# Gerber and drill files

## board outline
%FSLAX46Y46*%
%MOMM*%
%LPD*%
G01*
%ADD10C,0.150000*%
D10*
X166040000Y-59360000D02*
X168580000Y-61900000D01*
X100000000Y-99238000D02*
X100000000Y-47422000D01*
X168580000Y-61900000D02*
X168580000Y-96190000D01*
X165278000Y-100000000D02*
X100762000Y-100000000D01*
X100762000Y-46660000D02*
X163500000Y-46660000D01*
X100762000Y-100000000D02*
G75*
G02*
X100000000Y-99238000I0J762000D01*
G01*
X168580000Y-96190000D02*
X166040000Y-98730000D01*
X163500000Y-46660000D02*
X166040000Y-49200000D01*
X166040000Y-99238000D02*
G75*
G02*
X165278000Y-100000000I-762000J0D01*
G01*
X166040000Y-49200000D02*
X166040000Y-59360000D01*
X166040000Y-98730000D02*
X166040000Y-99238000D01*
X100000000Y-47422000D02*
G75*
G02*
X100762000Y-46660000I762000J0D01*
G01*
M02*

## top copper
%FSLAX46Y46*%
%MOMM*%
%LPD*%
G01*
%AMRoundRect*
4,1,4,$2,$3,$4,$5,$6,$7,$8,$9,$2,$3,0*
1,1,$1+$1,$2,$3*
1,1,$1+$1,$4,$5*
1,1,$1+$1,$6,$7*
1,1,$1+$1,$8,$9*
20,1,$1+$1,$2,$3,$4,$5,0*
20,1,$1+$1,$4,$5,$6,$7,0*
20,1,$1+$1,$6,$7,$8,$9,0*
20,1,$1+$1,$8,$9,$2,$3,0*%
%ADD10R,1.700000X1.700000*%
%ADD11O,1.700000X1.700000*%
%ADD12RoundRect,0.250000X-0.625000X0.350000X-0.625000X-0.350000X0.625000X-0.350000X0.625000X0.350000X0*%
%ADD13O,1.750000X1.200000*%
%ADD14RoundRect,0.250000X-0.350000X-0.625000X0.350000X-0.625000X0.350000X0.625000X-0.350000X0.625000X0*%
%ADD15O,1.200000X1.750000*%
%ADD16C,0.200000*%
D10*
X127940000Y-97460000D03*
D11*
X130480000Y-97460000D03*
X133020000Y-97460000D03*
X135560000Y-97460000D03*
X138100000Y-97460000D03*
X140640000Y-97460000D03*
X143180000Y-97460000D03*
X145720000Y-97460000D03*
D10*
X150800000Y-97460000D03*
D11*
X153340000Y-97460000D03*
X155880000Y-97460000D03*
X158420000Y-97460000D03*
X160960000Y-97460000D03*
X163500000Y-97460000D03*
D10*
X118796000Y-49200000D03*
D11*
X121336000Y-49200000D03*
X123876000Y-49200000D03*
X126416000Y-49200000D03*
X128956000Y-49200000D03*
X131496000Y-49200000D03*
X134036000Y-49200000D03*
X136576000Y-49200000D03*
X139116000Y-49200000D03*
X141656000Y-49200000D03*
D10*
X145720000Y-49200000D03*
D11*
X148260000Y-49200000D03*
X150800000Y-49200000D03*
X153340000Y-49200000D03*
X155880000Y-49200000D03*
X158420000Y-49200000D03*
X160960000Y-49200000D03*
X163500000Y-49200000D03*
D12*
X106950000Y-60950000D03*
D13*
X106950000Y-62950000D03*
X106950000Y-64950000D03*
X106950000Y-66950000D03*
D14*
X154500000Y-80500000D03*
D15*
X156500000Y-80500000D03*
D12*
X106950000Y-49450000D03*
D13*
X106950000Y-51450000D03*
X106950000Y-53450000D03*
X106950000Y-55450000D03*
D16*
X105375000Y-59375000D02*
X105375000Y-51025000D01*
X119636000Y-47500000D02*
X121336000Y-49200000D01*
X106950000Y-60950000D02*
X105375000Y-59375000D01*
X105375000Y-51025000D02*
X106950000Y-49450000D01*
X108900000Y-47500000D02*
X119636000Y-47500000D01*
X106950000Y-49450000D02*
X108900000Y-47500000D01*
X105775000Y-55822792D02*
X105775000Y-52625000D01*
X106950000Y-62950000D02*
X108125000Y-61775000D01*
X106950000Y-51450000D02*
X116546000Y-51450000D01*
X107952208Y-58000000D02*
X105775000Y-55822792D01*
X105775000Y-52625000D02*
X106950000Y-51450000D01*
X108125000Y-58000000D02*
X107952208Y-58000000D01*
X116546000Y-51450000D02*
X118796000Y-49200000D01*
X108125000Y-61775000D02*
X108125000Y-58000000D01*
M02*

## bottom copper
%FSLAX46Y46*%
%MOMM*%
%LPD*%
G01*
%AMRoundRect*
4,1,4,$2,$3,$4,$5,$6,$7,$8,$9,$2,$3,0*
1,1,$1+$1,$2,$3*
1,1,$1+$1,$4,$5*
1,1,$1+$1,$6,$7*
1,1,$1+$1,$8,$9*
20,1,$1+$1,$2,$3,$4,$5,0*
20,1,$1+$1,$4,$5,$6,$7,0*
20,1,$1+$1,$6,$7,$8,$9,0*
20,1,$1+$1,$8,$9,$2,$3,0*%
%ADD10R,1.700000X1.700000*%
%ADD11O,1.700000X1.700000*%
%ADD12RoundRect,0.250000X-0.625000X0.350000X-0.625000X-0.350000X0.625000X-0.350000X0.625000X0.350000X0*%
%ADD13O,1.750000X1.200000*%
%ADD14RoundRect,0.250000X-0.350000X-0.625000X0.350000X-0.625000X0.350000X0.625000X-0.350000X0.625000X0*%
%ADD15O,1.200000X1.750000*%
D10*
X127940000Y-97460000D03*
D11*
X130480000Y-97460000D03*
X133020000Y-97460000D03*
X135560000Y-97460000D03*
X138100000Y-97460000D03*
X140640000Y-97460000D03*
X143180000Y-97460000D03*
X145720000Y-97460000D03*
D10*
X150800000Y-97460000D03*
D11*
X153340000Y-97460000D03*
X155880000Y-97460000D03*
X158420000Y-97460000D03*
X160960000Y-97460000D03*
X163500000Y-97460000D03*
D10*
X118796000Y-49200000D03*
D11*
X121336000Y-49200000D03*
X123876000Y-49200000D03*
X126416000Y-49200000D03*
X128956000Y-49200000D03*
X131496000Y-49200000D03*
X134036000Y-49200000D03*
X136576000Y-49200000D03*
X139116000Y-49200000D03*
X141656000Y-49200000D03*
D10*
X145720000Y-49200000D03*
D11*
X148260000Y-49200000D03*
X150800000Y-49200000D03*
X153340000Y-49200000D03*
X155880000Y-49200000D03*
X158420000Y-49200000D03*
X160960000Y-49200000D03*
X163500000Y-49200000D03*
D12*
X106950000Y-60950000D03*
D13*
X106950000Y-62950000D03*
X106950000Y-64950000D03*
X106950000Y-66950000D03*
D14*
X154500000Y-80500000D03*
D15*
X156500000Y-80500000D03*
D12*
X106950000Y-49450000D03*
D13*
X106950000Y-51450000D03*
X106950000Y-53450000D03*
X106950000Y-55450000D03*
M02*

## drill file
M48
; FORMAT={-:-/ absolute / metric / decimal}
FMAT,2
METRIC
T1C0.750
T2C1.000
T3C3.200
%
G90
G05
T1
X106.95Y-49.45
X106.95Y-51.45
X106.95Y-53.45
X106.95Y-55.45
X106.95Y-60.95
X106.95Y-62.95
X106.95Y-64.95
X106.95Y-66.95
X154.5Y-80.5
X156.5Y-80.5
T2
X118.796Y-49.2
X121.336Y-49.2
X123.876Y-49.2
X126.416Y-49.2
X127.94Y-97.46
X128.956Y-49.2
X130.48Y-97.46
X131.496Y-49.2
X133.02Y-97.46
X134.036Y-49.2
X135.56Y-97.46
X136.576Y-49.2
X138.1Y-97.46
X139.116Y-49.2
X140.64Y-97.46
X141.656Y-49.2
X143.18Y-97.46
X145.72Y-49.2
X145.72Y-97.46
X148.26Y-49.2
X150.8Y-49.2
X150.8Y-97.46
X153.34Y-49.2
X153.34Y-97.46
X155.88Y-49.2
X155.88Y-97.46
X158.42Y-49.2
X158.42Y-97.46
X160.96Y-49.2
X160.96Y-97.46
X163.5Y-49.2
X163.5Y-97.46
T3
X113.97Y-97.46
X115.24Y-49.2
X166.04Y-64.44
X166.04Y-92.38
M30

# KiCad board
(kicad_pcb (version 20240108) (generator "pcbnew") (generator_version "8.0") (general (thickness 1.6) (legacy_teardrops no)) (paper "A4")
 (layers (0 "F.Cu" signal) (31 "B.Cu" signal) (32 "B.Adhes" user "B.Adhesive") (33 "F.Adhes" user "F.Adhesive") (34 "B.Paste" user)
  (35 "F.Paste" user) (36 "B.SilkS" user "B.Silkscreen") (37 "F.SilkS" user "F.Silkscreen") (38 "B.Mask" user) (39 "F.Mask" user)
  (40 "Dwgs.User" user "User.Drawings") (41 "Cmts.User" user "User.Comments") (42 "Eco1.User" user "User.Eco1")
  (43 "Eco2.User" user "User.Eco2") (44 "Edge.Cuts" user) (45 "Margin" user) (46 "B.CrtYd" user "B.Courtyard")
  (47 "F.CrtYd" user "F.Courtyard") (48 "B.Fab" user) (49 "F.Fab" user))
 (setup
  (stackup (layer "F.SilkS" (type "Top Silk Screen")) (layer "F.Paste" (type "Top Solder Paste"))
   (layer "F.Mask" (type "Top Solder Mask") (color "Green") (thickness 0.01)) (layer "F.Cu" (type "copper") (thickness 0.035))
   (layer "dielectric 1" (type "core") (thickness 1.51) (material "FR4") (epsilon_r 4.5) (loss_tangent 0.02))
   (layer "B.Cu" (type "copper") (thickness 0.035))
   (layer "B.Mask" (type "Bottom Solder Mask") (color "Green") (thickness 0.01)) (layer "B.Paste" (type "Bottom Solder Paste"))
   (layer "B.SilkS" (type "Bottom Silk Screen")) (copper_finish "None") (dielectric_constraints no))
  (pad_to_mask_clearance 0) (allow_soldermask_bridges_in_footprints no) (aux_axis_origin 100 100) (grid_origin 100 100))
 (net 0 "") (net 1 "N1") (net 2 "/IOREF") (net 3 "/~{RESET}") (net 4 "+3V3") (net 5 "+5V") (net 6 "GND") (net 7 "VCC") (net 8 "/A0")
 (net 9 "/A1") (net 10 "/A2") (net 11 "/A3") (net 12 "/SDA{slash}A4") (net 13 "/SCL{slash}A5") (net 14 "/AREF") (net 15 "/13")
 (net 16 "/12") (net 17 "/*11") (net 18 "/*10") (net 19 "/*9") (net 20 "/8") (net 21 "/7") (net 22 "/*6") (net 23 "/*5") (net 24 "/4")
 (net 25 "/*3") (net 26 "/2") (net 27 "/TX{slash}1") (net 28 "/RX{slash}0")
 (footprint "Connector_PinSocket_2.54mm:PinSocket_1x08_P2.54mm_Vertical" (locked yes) (layer "F.Cu") (at 127.94 97.46 90)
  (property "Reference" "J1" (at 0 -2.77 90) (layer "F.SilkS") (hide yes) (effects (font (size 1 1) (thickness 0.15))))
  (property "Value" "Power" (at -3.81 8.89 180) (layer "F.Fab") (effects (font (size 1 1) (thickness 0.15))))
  (pad "1" thru_hole rect (at 0 0 90) (size 1.7 1.7) (drill 1) (layers "*.Cu" "*.Mask") (remove_unused_layers no) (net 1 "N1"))
  (pad "2" thru_hole oval (at 0 2.54 90) (size 1.7 1.7) (drill 1) (layers "*.Cu" "*.Mask") (remove_unused_layers no) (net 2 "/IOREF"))
  (pad "3" thru_hole oval (at 0 5.08 90) (size 1.7 1.7) (drill 1) (layers "*.Cu" "*.Mask") (remove_unused_layers no) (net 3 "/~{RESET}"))
  (pad "4" thru_hole oval (at 0 7.62 90) (size 1.7 1.7) (drill 1) (layers "*.Cu" "*.Mask") (remove_unused_layers no) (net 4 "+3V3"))
  (pad "5" thru_hole oval (at 0 10.16 90) (size 1.7 1.7) (drill 1) (layers "*.Cu" "*.Mask") (remove_unused_layers no) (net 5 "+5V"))
  (pad "6" thru_hole oval (at 0 12.7 90) (size 1.7 1.7) (drill 1) (layers "*.Cu" "*.Mask") (remove_unused_layers no) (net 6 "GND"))
  (pad "7" thru_hole oval (at 0 15.24 90) (size 1.7 1.7) (drill 1) (layers "*.Cu" "*.Mask") (remove_unused_layers no) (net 6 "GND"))
  (pad "8" thru_hole oval (at 0 17.78 90) (size 1.7 1.7) (drill 1) (layers "*.Cu" "*.Mask") (remove_unused_layers no) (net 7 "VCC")))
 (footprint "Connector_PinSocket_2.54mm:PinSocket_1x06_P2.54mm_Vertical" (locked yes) (layer "F.Cu") (at 150.8 97.46 90)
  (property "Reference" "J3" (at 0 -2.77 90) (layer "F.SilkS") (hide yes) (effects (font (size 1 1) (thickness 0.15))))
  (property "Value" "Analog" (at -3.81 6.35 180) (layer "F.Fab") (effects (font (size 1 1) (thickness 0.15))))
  (pad "1" thru_hole rect (at 0 0 90) (size 1.7 1.7) (drill 1) (layers "*.Cu" "*.Mask") (remove_unused_layers no) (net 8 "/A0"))
  (pad "2" thru_hole oval (at 0 2.54 90) (size 1.7 1.7) (drill 1) (layers "*.Cu" "*.Mask") (remove_unused_layers no) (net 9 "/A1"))
  (pad "3" thru_hole oval (at 0 5.08 90) (size 1.7 1.7) (drill 1) (layers "*.Cu" "*.Mask") (remove_unused_layers no) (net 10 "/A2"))
  (pad "4" thru_hole oval (at 0 7.62 90) (size 1.7 1.7) (drill 1) (layers "*.Cu" "*.Mask") (remove_unused_layers no) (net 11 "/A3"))
  (pad "5" thru_hole oval (at 0 10.16 90) (size 1.7 1.7) (drill 1) (layers "*.Cu" "*.Mask") (remove_unused_layers no)
   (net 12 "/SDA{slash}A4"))
  (pad "6" thru_hole oval (at 0 12.7 90) (size 1.7 1.7) (drill 1) (layers "*.Cu" "*.Mask") (remove_unused_layers no)
   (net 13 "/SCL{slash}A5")))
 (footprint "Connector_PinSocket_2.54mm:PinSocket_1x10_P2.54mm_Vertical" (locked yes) (layer "F.Cu") (at 118.796 49.2 90)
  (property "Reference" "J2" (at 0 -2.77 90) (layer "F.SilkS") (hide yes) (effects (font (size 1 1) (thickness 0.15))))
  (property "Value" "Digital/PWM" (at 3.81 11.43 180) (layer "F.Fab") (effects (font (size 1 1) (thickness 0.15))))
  (pad "1" thru_hole rect (at 0 0 90) (size 1.7 1.7) (drill 1) (layers "*.Cu" "*.Mask") (remove_unused_layers no) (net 13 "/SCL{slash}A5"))
  (pad "2" thru_hole oval (at 0 2.54 90) (size 1.7 1.7) (drill 1) (layers "*.Cu" "*.Mask") (remove_unused_layers no)
   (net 12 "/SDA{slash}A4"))
  (pad "3" thru_hole oval (at 0 5.08 90) (size 1.7 1.7) (drill 1) (layers "*.Cu" "*.Mask") (remove_unused_layers no) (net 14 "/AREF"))
  (pad "4" thru_hole oval (at 0 7.62 90) (size 1.7 1.7) (drill 1) (layers "*.Cu" "*.Mask") (remove_unused_layers no) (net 6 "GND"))
  (pad "5" thru_hole oval (at 0 10.16 90) (size 1.7 1.7) (drill 1) (layers "*.Cu" "*.Mask") (remove_unused_layers no) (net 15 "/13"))
  (pad "6" thru_hole oval (at 0 12.7 90) (size 1.7 1.7) (drill 1) (layers "*.Cu" "*.Mask") (remove_unused_layers no) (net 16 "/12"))
  (pad "7" thru_hole oval (at 0 15.24 90) (size 1.7 1.7) (drill 1) (layers "*.Cu" "*.Mask") (remove_unused_layers no) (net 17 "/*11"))
  (pad "8" thru_hole oval (at 0 17.78 90) (size 1.7 1.7) (drill 1) (layers "*.Cu" "*.Mask") (remove_unused_layers no) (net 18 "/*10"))
  (pad "9" thru_hole oval (at 0 20.32 90) (size 1.7 1.7) (drill 1) (layers "*.Cu" "*.Mask") (remove_unused_layers no) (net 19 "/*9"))
  (pad "10" thru_hole oval (at 0 22.86 90) (size 1.7 1.7) (drill 1) (layers "*.Cu" "*.Mask") (remove_unused_layers no) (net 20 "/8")))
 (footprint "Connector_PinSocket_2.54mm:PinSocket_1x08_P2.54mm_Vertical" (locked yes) (layer "F.Cu") (at 145.72 49.2 90)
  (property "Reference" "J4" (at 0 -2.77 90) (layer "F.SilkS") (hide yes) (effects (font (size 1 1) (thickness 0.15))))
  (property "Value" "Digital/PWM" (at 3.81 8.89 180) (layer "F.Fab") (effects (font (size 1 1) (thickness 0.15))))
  (pad "1" thru_hole rect (at 0 0 90) (size 1.7 1.7) (drill 1) (layers "*.Cu" "*.Mask") (remove_unused_layers no) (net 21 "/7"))
  (pad "2" thru_hole oval (at 0 2.54 90) (size 1.7 1.7) (drill 1) (layers "*.Cu" "*.Mask") (remove_unused_layers no) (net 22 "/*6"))
  (pad "3" thru_hole oval (at 0 5.08 90) (size 1.7 1.7) (drill 1) (layers "*.Cu" "*.Mask") (remove_unused_layers no) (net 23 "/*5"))
  (pad "4" thru_hole oval (at 0 7.62 90) (size 1.7 1.7) (drill 1) (layers "*.Cu" "*.Mask") (remove_unused_layers no) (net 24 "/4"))
  (pad "5" thru_hole oval (at 0 10.16 90) (size 1.7 1.7) (drill 1) (layers "*.Cu" "*.Mask") (remove_unused_layers no) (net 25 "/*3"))
  (pad "6" thru_hole oval (at 0 12.7 90) (size 1.7 1.7) (drill 1) (layers "*.Cu" "*.Mask") (remove_unused_layers no) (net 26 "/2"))
  (pad "7" thru_hole oval (at 0 15.24 90) (size 1.7 1.7) (drill 1) (layers "*.Cu" "*.Mask") (remove_unused_layers no) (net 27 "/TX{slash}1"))
  (pad "8" thru_hole oval (at 0 17.78 90) (size 1.7 1.7) (drill 1) (layers "*.Cu" "*.Mask") (remove_unused_layers no) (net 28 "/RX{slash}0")))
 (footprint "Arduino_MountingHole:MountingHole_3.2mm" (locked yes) (layer "F.Cu") (at 115.24 49.2)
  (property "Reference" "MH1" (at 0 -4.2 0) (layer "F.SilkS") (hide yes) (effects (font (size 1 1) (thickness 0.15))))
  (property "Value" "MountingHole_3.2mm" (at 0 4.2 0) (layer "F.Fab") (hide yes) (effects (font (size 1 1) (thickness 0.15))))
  (pad "" np_thru_hole circle (at 0 0) (size 3.2 3.2) (drill 3.2) (layers "*.Cu" "*.Mask")))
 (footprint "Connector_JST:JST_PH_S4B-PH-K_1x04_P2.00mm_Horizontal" (layer "F.Cu") (at 106.95 60.95 -90)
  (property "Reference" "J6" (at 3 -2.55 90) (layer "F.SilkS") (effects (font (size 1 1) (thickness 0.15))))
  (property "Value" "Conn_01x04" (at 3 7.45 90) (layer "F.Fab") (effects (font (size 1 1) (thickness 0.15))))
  (pad "1" thru_hole roundrect (at 0 0 270) (size 1.2 1.75) (drill 0.75) (layers "*.Cu" "*.Mask") (remove_unused_layers no)
   (roundrect_rratio 0.208333) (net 12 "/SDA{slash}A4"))
  (pad "2" thru_hole oval (at 2 0 270) (size 1.2 1.75) (drill 0.75) (layers "*.Cu" "*.Mask") (remove_unused_layers no)
   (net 13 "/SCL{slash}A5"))
  (pad "3" thru_hole oval (at 4 0 270) (size 1.2 1.75) (drill 0.75) (layers "*.Cu" "*.Mask") (remove_unused_layers no) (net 7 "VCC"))
  (pad "4" thru_hole oval (at 6 0 270) (size 1.2 1.75) (drill 0.75) (layers "*.Cu" "*.Mask") (remove_unused_layers no) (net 6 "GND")))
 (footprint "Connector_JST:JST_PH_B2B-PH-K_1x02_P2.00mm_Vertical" (layer "F.Cu") (at 154.5 80.5)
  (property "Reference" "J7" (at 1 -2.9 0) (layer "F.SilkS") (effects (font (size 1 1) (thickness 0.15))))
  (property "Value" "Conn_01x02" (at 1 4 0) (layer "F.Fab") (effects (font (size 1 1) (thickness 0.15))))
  (pad "1" thru_hole roundrect (at 0 0) (size 1.2 1.75) (drill 0.75) (layers "*.Cu" "*.Mask") (remove_unused_layers no)
   (roundrect_rratio 0.208333) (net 6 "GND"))
  (pad "2" thru_hole oval (at 2 0) (size 1.2 1.75) (drill 0.75) (layers "*.Cu" "*.Mask") (remove_unused_layers no) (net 7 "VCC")))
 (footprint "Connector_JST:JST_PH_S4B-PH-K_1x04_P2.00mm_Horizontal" (layer "F.Cu") (at 106.95 49.45 -90)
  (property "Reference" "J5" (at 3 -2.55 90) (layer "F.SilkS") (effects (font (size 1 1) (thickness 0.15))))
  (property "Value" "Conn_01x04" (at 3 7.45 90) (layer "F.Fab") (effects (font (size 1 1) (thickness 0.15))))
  (pad "1" thru_hole roundrect (at 0 0 270) (size 1.2 1.75) (drill 0.75) (layers "*.Cu" "*.Mask") (remove_unused_layers no)
   (roundrect_rratio 0.208333) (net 12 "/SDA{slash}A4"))
  (pad "2" thru_hole oval (at 2 0 270) (size 1.2 1.75) (drill 0.75) (layers "*.Cu" "*.Mask") (remove_unused_layers no)
   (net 13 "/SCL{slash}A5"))
  (pad "3" thru_hole oval (at 4 0 270) (size 1.2 1.75) (drill 0.75) (layers "*.Cu" "*.Mask") (remove_unused_layers no) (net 7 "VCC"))
  (pad "4" thru_hole oval (at 6 0 270) (size 1.2 1.75) (drill 0.75) (layers "*.Cu" "*.Mask") (remove_unused_layers no) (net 6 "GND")))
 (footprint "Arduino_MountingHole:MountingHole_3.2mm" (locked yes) (layer "F.Cu") (at 113.97 97.46)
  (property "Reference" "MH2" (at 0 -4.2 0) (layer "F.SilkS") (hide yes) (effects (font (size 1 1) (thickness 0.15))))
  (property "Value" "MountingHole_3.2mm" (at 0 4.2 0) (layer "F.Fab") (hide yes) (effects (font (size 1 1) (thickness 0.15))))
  (pad "" np_thru_hole circle (at 0 0) (size 3.2 3.2) (drill 3.2) (layers "*.Cu" "*.Mask")))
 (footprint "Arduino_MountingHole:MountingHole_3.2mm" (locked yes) (layer "F.Cu") (at 166.04 64.44)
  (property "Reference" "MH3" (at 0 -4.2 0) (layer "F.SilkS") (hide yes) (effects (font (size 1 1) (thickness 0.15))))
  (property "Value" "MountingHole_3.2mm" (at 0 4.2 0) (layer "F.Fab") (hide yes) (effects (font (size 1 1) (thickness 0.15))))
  (pad "" np_thru_hole circle (at 0 0) (size 3.2 3.2) (drill 3.2) (layers "*.Cu" "*.Mask")))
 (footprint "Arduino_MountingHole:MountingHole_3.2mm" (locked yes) (layer "F.Cu") (at 166.04 92.38)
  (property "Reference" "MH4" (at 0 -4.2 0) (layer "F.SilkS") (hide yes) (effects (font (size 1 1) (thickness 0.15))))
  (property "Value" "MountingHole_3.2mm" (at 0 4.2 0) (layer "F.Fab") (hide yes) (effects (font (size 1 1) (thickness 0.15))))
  (pad "" np_thru_hole circle (at 0 0) (size 3.2 3.2) (drill 3.2) (layers "*.Cu" "*.Mask")))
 (gr_line (start 166.04 59.36) (end 168.58 61.9) (stroke (width 0.15) (type solid)) (layer "Edge.Cuts"))
 (gr_line (start 100 99.238) (end 100 47.422) (stroke (width 0.15) (type solid)) (layer "Edge.Cuts"))
 (gr_line (start 168.58 61.9) (end 168.58 96.19) (stroke (width 0.15) (type solid)) (layer "Edge.Cuts"))
 (gr_line (start 165.278 100) (end 100.762 100) (stroke (width 0.15) (type solid)) (layer "Edge.Cuts"))
 (gr_line (start 100.762 46.66) (end 163.5 46.66) (stroke (width 0.15) (type solid)) (layer "Edge.Cuts"))
 (gr_arc (start 100.762 100) (mid 100.223185 99.776815) (end 100 99.238) (stroke (width 0.15) (type solid)) (layer "Edge.Cuts"))
 (gr_line (start 168.58 96.19) (end 166.04 98.73) (stroke (width 0.15) (type solid)) (layer "Edge.Cuts"))
 (gr_line (start 163.5 46.66) (end 166.04 49.2) (stroke (width 0.15) (type solid)) (layer "Edge.Cuts"))
 (gr_arc (start 166.04 99.238) (mid 165.816815 99.776815) (end 165.278 100) (stroke (width 0.15) (type solid)) (layer "Edge.Cuts"))
 (gr_line (start 166.04 49.2) (end 166.04 59.36) (stroke (width 0.15) (type solid)) (layer "Edge.Cuts"))
 (gr_line (start 166.04 98.73) (end 166.04 99.238) (stroke (width 0.15) (type solid)) (layer "Edge.Cuts"))
 (gr_arc (start 100 47.422) (mid 100.223185 46.883185) (end 100.762 46.66) (stroke (width 0.15) (type solid)) (layer "Edge.Cuts"))
 (segment (start 105.375 59.375) (end 105.375 51.025) (width 0.2) (layer "F.Cu") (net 12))
 (segment (start 119.636 47.5) (end 121.336 49.2) (width 0.2) (layer "F.Cu") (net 12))
 (segment (start 106.95 60.95) (end 105.375 59.375) (width 0.2) (layer "F.Cu") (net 12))
 (segment (start 105.375 51.025) (end 106.95 49.45) (width 0.2) (layer "F.Cu") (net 12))
 (segment (start 108.9 47.5) (end 119.636 47.5) (width 0.2) (layer "F.Cu") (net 12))
 (segment (start 106.95 49.45) (end 108.9 47.5) (width 0.2) (layer "F.Cu") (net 12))
 (segment (start 105.775 55.822792) (end 105.775 52.625) (width 0.2) (layer "F.Cu") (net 13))
 (segment (start 106.95 62.95) (end 108.125 61.775) (width 0.2) (layer "F.Cu") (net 13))
 (segment (start 106.95 51.45) (end 116.546 51.45) (width 0.2) (layer "F.Cu") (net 13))
 (segment (start 107.952208 58) (end 105.775 55.822792) (width 0.2) (layer "F.Cu") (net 13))
 (segment (start 105.775 52.625) (end 106.95 51.45) (width 0.2) (layer "F.Cu") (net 13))
 (segment (start 108.125 58) (end 107.952208 58) (width 0.2) (layer "F.Cu") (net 13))
 (segment (start 116.546 51.45) (end 118.796 49.2) (width 0.2) (layer "F.Cu") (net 13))
 (segment (start 108.125 61.775) (end 108.125 58) (width 0.2) (layer "F.Cu") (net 13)))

